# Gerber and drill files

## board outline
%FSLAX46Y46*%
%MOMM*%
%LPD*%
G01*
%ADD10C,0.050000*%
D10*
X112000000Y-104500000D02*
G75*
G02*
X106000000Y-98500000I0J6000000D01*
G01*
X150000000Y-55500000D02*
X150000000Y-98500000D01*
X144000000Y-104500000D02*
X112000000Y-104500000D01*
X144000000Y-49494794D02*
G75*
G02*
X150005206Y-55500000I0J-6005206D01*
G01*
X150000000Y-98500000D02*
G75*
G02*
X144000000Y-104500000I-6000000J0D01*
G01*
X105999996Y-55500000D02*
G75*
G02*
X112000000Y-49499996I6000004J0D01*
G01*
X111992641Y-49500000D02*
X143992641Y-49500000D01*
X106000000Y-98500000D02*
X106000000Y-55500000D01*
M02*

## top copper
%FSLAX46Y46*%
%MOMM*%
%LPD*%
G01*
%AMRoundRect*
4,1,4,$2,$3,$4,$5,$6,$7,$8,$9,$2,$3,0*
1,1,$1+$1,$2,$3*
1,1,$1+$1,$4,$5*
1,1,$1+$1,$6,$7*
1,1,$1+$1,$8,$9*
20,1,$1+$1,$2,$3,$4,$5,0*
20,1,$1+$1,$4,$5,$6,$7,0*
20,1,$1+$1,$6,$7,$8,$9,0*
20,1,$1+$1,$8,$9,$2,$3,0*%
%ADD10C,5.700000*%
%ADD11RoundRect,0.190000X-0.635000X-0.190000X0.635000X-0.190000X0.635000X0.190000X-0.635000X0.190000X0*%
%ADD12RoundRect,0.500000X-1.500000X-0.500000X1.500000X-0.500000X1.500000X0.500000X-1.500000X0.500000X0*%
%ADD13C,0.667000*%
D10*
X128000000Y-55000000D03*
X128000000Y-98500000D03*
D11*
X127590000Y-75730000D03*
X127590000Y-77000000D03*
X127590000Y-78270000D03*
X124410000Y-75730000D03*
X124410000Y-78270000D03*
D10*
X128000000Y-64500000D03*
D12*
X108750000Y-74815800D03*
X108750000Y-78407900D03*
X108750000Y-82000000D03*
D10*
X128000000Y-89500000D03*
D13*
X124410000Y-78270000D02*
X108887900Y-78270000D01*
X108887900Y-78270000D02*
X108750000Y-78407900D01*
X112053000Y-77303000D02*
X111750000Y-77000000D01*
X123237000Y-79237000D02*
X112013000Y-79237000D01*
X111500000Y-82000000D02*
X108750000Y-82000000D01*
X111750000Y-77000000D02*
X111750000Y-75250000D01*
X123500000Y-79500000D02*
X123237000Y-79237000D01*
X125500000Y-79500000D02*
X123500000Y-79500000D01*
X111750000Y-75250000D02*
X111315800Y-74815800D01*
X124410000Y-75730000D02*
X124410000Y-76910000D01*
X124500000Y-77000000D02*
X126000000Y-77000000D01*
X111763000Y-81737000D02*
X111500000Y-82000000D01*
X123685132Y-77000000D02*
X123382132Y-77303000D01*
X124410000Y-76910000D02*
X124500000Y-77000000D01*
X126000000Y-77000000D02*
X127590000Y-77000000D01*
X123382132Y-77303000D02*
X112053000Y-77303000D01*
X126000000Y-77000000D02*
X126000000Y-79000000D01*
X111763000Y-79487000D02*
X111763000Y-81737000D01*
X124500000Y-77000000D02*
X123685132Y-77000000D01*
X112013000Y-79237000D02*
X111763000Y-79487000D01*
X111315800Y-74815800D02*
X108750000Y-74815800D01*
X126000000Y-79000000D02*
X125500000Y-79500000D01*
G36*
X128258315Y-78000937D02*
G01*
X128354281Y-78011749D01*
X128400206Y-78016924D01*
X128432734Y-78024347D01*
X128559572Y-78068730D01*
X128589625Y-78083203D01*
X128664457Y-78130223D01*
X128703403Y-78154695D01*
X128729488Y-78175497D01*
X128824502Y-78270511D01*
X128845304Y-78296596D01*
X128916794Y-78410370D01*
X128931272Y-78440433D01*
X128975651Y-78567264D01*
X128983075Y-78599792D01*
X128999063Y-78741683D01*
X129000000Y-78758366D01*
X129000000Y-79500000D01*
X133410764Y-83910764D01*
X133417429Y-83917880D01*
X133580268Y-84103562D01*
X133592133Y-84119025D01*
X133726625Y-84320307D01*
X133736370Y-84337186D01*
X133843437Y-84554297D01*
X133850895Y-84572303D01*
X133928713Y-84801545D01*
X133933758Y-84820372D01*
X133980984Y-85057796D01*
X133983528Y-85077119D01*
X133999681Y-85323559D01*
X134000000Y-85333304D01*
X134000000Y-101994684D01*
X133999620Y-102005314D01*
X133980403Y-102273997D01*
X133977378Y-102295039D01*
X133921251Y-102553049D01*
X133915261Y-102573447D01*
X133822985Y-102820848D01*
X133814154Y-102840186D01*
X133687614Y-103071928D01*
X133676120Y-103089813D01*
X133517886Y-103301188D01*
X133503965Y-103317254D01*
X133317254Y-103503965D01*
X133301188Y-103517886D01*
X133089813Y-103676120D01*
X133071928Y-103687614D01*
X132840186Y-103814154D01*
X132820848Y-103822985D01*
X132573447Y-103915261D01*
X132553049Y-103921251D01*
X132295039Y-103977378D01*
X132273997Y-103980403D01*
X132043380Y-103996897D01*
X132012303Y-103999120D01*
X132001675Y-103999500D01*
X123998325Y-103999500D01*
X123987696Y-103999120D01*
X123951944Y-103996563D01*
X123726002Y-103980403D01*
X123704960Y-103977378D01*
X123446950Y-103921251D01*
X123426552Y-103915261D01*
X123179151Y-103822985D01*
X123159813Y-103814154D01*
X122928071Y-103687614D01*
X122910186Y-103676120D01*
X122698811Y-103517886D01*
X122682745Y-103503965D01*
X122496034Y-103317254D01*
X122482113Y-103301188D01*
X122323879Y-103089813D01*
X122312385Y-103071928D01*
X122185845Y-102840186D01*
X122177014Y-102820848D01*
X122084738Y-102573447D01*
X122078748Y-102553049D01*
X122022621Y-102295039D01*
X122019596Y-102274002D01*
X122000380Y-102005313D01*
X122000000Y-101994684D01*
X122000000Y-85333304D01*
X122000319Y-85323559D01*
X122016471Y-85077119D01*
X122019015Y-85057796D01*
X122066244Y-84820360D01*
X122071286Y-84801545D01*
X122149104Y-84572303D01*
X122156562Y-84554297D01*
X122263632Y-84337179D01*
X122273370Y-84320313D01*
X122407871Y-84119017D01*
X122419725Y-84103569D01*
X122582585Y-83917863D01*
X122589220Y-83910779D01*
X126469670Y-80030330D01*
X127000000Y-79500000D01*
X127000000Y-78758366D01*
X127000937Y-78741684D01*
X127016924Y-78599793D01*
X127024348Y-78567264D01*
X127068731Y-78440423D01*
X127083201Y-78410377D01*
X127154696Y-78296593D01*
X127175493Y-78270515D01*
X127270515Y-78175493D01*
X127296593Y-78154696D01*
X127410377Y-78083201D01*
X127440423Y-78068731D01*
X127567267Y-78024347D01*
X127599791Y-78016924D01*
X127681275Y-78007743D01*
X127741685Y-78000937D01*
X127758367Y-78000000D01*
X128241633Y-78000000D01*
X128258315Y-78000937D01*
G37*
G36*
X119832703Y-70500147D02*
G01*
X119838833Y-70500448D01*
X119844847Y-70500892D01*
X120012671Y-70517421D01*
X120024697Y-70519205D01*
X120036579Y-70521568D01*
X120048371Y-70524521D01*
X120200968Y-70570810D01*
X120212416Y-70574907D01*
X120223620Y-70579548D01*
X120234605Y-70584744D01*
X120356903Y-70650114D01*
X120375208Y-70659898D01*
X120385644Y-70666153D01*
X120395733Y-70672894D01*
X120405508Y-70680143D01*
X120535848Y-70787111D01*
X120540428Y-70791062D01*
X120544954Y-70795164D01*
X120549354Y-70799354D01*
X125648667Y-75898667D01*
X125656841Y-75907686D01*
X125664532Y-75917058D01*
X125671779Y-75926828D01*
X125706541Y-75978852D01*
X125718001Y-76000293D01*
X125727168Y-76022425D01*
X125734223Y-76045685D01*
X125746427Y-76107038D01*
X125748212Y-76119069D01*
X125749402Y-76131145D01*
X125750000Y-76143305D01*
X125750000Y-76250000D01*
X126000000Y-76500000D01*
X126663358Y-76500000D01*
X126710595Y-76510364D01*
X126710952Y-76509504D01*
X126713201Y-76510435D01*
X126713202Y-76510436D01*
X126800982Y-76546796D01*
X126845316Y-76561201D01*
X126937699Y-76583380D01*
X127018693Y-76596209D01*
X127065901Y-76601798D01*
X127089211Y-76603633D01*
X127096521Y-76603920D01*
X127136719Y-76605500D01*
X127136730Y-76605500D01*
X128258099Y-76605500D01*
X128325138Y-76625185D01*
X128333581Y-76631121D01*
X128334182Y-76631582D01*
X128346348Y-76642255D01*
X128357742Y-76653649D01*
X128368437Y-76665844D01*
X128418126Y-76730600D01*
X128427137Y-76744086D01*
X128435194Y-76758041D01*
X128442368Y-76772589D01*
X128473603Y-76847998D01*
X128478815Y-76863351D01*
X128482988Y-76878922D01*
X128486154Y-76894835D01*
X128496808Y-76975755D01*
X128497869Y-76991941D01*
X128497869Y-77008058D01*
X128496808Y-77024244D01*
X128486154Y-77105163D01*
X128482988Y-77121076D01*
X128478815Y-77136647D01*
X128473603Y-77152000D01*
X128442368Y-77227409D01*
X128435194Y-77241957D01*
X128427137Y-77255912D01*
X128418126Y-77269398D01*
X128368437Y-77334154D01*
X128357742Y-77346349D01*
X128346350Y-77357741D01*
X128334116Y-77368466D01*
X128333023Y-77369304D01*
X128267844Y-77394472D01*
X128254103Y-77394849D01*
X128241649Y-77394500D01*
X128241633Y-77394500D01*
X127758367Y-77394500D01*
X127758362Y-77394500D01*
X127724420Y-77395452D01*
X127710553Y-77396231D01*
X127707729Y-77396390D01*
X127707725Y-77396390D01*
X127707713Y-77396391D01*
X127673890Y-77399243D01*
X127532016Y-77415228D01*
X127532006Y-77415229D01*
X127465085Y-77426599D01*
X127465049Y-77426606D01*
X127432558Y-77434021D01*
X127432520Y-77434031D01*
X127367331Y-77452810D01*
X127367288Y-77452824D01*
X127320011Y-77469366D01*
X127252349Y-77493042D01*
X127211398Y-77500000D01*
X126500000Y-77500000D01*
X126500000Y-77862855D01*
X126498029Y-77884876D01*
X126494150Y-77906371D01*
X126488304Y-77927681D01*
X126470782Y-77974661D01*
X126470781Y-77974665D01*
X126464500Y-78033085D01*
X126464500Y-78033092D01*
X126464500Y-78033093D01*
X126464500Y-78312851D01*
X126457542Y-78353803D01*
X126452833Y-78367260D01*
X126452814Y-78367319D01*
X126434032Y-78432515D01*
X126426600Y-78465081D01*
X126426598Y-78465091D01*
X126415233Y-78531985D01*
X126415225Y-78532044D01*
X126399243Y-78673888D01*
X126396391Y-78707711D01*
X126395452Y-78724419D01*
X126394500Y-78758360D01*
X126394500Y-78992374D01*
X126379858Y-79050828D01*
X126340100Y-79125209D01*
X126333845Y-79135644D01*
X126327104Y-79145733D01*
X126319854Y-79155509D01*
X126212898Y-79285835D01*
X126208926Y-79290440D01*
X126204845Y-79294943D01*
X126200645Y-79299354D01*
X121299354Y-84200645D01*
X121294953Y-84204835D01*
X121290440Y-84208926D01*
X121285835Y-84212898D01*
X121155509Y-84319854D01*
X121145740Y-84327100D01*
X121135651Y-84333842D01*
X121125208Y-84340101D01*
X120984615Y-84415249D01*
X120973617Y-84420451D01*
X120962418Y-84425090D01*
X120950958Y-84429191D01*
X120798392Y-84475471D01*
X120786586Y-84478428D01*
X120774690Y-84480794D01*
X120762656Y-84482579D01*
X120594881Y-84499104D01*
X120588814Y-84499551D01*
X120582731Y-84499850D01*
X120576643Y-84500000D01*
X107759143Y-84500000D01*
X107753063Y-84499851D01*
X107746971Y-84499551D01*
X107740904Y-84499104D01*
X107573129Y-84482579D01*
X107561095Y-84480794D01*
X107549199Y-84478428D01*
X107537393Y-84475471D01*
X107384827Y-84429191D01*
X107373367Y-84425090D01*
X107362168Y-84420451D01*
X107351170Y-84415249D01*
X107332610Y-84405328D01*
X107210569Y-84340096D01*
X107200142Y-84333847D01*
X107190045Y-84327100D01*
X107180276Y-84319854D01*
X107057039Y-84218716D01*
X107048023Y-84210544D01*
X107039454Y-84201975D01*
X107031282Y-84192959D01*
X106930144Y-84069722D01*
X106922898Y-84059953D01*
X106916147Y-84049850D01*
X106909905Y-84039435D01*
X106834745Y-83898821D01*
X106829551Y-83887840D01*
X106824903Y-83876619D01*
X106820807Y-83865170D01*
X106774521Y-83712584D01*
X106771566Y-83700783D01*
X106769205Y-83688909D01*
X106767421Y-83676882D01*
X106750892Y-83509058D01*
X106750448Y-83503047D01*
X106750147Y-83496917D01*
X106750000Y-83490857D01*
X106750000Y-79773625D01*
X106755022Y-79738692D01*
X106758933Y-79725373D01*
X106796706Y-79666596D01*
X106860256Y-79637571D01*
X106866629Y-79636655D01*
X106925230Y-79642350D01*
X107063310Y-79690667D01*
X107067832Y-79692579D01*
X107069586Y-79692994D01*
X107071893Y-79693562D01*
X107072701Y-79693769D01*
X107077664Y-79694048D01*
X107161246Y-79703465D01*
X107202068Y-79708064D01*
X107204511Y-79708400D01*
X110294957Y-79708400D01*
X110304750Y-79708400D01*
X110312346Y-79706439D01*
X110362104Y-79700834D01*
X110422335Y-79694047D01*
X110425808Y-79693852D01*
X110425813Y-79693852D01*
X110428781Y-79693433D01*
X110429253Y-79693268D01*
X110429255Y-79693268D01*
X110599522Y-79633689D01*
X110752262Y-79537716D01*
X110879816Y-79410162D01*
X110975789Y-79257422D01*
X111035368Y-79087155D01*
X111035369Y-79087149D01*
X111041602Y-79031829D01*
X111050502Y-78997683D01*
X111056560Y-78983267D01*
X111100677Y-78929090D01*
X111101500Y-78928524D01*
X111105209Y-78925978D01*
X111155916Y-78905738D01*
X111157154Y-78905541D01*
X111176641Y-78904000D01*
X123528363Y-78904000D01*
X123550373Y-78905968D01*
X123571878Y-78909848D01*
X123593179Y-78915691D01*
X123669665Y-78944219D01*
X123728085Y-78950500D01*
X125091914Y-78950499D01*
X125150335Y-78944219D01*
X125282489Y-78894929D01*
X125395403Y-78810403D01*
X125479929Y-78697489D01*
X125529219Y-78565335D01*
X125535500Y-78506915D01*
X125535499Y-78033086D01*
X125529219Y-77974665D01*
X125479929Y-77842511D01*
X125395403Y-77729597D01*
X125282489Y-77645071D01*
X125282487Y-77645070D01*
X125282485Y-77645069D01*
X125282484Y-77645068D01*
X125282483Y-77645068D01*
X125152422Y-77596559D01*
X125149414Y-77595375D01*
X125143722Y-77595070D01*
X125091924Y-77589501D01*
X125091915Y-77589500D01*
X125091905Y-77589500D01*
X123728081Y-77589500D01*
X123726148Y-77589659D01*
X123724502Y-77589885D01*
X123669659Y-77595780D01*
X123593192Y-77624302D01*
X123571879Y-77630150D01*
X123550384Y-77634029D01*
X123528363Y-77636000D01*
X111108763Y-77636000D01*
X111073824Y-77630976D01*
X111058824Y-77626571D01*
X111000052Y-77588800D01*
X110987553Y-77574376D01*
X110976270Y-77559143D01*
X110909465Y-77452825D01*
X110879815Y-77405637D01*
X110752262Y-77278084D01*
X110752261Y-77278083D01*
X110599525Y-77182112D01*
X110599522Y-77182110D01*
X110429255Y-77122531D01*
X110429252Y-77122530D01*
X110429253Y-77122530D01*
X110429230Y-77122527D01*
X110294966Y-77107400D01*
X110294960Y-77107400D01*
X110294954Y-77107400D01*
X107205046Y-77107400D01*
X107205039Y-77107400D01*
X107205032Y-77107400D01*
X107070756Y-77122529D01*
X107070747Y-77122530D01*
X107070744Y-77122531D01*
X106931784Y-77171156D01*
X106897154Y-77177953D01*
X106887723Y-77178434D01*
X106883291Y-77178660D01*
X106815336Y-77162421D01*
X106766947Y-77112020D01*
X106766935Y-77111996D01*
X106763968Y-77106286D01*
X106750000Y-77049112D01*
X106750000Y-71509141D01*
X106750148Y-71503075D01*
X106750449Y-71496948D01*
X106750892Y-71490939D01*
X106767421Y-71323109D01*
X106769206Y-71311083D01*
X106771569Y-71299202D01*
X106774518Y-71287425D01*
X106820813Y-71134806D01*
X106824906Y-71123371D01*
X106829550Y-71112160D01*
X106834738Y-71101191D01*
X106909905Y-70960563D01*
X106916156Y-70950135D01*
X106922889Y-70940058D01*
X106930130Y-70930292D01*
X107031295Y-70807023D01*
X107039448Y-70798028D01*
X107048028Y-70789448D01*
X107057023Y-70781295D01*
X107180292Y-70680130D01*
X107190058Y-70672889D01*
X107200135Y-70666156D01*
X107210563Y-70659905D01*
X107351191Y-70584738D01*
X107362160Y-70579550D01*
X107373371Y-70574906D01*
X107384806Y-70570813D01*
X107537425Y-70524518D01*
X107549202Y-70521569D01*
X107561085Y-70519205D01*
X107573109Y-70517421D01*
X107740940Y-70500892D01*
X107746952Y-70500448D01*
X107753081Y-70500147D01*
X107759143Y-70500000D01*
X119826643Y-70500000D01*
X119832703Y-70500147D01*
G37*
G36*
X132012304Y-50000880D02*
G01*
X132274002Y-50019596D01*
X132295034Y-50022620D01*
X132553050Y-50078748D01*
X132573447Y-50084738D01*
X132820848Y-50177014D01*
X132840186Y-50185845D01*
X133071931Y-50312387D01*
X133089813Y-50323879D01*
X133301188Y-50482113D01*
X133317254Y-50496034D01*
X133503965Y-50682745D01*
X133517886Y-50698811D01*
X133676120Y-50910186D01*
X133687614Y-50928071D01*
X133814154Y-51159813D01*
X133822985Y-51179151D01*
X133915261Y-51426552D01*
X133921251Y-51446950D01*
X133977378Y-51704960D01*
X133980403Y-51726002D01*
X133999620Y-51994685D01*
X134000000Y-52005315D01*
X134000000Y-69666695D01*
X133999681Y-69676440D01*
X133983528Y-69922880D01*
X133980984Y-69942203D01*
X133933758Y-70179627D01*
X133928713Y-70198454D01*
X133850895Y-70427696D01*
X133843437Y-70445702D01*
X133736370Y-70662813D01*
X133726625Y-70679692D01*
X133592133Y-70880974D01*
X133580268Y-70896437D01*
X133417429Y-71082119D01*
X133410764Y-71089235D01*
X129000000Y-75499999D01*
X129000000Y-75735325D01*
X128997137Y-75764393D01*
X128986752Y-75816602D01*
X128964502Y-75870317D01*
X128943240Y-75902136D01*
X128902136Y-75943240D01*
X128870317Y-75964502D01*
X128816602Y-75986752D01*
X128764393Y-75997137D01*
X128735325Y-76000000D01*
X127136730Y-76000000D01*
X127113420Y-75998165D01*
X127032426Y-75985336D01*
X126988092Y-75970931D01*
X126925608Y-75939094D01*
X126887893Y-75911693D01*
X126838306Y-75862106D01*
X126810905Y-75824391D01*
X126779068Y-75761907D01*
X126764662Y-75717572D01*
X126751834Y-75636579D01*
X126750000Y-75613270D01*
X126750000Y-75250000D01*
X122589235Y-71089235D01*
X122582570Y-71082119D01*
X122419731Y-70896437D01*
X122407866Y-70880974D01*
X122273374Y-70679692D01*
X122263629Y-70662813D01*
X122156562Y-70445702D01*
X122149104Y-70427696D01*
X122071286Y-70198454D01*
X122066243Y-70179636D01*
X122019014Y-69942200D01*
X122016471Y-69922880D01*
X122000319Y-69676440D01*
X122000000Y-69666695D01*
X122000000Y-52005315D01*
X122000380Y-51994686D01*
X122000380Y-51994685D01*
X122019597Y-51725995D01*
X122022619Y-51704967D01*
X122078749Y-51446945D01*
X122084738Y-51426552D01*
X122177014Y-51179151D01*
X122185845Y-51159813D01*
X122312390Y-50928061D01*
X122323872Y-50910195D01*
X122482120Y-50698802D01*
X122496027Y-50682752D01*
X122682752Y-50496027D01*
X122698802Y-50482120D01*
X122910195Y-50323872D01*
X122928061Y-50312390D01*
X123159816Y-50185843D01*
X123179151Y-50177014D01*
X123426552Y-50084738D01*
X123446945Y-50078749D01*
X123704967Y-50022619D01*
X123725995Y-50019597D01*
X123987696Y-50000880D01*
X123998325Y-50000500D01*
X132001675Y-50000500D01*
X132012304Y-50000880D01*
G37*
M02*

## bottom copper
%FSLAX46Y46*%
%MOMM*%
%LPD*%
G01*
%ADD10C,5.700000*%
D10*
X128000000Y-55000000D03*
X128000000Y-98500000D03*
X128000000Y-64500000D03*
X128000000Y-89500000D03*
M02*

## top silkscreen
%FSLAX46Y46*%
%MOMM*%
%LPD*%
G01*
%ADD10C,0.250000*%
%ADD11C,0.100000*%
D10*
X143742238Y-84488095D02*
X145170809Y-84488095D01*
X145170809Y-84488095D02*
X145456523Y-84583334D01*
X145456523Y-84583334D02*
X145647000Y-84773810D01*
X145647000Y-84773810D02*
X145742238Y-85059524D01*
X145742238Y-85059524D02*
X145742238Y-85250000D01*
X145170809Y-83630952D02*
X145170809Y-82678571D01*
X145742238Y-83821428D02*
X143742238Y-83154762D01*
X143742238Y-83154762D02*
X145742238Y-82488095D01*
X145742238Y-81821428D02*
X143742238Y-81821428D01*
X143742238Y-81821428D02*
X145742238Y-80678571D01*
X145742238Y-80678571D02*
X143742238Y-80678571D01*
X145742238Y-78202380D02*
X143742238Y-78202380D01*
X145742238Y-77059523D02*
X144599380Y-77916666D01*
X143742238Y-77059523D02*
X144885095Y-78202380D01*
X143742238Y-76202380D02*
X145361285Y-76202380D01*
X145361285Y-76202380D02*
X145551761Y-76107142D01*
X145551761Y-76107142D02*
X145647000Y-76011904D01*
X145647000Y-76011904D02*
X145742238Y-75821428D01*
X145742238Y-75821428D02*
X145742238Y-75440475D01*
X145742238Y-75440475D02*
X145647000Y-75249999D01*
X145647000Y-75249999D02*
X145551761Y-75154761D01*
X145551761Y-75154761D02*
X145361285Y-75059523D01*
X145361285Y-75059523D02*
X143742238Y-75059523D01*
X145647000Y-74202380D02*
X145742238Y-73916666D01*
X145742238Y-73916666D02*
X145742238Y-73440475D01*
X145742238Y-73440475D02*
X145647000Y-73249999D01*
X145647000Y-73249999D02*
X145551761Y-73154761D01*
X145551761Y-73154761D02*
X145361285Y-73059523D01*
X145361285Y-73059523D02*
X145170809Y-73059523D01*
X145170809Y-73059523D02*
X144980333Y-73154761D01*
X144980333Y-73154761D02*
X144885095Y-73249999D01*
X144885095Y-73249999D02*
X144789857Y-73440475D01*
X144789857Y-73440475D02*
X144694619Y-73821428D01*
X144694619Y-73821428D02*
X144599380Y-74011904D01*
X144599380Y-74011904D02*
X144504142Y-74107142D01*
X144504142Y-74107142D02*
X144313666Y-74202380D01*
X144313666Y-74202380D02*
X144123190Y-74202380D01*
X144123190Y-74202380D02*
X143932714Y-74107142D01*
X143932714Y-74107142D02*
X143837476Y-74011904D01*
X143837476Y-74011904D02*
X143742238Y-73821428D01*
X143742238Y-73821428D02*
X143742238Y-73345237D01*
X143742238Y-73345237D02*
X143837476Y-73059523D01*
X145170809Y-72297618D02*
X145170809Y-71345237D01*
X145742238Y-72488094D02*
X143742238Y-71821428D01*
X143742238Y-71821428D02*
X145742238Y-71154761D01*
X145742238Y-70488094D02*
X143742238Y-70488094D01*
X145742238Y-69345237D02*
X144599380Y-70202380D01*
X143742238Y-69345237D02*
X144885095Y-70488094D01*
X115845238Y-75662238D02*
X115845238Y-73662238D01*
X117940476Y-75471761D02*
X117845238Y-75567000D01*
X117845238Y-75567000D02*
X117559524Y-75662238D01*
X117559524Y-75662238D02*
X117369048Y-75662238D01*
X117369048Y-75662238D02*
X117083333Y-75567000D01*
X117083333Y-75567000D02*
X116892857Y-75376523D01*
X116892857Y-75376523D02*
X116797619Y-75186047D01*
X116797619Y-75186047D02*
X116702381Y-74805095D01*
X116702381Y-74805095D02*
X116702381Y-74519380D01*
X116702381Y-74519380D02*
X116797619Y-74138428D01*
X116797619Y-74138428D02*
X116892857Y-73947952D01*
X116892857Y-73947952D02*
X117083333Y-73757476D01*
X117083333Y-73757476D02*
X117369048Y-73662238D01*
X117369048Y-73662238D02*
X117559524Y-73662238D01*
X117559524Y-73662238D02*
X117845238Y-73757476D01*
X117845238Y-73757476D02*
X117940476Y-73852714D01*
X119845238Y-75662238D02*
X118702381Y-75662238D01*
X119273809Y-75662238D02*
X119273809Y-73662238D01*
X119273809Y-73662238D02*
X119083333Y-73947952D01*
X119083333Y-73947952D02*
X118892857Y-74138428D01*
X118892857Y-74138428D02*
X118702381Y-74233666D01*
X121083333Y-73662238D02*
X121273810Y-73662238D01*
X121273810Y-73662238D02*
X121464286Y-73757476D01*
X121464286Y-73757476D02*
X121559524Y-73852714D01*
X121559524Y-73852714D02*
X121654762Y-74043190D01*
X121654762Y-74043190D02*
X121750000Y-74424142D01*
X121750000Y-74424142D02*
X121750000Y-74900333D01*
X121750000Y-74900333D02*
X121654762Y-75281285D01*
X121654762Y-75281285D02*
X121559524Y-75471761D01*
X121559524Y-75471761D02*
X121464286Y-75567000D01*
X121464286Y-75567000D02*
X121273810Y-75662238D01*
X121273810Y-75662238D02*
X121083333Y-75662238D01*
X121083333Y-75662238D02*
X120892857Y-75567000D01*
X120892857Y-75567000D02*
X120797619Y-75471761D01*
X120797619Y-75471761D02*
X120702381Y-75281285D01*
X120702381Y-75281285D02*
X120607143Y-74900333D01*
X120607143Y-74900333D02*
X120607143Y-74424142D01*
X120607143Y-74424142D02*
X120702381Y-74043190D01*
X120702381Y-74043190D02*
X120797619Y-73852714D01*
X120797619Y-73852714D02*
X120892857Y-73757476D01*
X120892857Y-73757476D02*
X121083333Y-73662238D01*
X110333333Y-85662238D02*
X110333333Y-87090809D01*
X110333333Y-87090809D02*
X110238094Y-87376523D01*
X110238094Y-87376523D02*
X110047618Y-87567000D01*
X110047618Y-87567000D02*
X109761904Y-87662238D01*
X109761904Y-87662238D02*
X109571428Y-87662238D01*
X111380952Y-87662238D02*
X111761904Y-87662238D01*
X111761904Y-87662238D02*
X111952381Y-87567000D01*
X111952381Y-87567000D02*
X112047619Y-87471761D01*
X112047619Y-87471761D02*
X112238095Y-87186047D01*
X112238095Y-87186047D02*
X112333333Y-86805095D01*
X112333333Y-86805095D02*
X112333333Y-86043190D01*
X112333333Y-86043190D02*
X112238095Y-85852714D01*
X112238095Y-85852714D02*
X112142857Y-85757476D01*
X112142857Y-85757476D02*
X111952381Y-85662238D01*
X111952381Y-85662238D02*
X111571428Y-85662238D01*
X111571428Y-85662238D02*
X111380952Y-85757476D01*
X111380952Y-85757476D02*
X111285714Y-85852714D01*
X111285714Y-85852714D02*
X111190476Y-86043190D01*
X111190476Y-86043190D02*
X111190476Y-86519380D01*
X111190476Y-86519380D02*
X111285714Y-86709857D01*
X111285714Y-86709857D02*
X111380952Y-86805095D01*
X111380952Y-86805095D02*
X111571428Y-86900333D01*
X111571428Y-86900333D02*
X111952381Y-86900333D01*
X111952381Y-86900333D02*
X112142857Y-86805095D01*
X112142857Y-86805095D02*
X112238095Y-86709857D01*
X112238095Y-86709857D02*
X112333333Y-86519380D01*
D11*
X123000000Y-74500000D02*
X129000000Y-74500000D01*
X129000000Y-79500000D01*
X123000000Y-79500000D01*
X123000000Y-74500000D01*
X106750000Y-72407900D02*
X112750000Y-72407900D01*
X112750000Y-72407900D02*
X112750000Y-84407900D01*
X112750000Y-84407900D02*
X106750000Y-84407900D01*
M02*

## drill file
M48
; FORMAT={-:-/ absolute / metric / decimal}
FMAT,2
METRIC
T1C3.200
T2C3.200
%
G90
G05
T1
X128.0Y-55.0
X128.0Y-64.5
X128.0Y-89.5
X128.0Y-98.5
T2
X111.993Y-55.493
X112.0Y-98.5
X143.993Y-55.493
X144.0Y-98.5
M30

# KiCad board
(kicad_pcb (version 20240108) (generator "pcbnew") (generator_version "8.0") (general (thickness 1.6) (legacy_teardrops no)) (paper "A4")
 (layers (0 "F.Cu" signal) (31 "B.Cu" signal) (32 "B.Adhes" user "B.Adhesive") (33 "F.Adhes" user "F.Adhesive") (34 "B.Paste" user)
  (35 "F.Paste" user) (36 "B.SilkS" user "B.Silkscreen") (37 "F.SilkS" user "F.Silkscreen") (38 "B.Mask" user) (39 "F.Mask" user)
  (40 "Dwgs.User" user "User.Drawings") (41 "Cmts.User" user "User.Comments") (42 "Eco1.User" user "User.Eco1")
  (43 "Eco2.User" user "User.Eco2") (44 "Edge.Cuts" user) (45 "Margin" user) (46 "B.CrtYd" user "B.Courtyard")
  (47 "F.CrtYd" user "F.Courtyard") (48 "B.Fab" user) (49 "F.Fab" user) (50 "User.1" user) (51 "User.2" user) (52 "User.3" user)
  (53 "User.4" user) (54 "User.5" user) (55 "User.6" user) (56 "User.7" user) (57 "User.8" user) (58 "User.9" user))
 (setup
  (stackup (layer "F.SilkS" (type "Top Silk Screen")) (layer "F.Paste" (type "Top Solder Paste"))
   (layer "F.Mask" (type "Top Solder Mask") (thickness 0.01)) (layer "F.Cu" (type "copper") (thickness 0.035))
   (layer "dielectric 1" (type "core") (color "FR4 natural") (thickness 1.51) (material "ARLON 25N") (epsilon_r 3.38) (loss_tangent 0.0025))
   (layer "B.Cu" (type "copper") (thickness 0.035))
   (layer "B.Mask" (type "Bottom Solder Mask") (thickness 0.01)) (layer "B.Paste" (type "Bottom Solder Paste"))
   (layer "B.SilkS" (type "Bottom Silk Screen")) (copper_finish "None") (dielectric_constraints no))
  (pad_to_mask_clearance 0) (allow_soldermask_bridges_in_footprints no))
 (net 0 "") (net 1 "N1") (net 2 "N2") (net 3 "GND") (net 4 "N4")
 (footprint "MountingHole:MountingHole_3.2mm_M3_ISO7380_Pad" (layer "F.Cu") (at 128 55)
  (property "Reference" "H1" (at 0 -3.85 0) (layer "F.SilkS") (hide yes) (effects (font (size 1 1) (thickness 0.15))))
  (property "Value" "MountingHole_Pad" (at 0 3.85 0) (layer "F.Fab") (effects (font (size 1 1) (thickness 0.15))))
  (pad "1" thru_hole circle (at 0 0) (size 5.7 5.7) (drill 3.2) (layers "*.Cu" "*.Mask") (remove_unused_layers no) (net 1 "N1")))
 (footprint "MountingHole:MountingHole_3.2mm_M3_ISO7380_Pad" (layer "F.Cu") (at 128 98.5)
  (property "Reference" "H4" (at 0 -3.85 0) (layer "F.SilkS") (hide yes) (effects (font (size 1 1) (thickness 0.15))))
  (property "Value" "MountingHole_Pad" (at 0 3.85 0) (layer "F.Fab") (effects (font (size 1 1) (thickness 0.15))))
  (pad "1" thru_hole circle (at 0 0) (size 5.7 5.7) (drill 3.2) (layers "*.Cu" "*.Mask") (remove_unused_layers no) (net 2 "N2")))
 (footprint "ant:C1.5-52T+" (layer "F.Cu") (at 126 77 -90)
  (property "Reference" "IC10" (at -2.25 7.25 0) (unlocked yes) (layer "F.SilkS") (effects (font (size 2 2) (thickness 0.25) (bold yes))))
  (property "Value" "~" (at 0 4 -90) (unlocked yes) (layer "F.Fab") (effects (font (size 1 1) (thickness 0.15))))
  (fp_rect (start -2.5 -3) (end 2.5 3) (stroke (width 0.1) (type default)) (fill none) (layer "F.SilkS"))
  (pad "1" smd roundrect (at -1.27 -1.59) (size 1.65 0.76) (layers "F.Cu" "F.Paste" "F.Mask") (roundrect_rratio 0.25) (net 1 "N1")
   (thermal_bridge_angle 45))
  (pad "2" smd roundrect (at 0 -1.59) (size 1.65 0.76) (layers "F.Cu" "F.Paste" "F.Mask") (roundrect_rratio 0.25) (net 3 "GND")
   (thermal_bridge_angle 45))
  (pad "3" smd roundrect (at 1.27 -1.59) (size 1.65 0.76) (layers "F.Cu" "F.Paste" "F.Mask") (roundrect_rratio 0.25) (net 2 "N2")
   (thermal_bridge_angle 45))
  (pad "4" smd roundrect (at -1.27 1.59) (size 1.65 0.76) (layers "F.Cu" "F.Paste" "F.Mask") (roundrect_rratio 0.25) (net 3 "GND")
   (thermal_bridge_angle 45))
  (pad "6" smd roundrect (at 1.27 1.59) (size 1.65 0.76) (layers "F.Cu" "F.Paste" "F.Mask") (roundrect_rratio 0.25) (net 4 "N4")
   (thermal_bridge_angle 45)))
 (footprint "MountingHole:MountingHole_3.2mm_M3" (layer "F.Cu") (at 112 98.5)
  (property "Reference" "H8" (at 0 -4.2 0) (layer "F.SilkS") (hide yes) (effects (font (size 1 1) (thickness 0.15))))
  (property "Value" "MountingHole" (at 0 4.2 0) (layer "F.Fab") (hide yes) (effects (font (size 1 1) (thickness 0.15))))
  (pad "" np_thru_hole circle (at 0 0) (size 3.2 3.2) (drill 3.2) (layers "*.Cu" "*.Mask")))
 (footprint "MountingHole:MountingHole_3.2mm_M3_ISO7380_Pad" (layer "F.Cu") (at 128 64.5)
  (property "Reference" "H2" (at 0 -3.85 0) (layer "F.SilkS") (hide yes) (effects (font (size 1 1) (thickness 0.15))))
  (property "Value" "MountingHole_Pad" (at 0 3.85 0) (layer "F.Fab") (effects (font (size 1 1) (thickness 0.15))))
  (pad "1" thru_hole circle (at 0 0) (size 5.7 5.7) (drill 3.2) (layers "*.Cu" "*.Mask") (remove_unused_layers no) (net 1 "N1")))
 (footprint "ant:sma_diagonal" (layer "F.Cu") (at 108.75 78.4079)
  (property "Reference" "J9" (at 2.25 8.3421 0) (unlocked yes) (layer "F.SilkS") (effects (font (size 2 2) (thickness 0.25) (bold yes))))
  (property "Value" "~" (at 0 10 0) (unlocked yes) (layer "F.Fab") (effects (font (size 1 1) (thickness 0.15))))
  (fp_line (start -2 -6) (end 4 -6) (stroke (width 0.1) (type default)) (layer "F.SilkS"))
  (fp_line (start 4 -6) (end 4 6) (stroke (width 0.1) (type default)) (layer "F.SilkS"))
  (fp_line (start 4 6) (end -2 6) (stroke (width 0.1) (type default)) (layer "F.SilkS"))
  (pad "1" smd roundrect (at 0 -3.5921) (size 4 2) (layers "F.Cu" "F.Paste" "F.Mask") (roundrect_rratio 0.25) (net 3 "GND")
   (thermal_bridge_angle 45))
  (pad "2" smd roundrect (at 0 0) (size 4 2) (layers "F.Cu" "F.Paste" "F.Mask") (roundrect_rratio 0.25) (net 4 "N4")
   (thermal_bridge_angle 45))
  (pad "3" smd roundrect (at 0 3.5921) (size 4 2) (layers "F.Cu" "F.Paste" "F.Mask") (roundrect_rratio 0.25) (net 3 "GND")
   (thermal_bridge_angle 45)))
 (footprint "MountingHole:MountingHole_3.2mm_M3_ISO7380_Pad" (layer "F.Cu") (at 128 89.5)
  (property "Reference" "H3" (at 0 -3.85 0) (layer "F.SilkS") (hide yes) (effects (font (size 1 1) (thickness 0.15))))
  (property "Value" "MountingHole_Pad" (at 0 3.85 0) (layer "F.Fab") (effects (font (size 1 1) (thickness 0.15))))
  (pad "1" thru_hole circle (at 0 0) (size 5.7 5.7) (drill 3.2) (layers "*.Cu" "*.Mask") (remove_unused_layers no) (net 2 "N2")))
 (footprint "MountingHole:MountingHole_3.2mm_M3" (layer "F.Cu") (at 144 98.5)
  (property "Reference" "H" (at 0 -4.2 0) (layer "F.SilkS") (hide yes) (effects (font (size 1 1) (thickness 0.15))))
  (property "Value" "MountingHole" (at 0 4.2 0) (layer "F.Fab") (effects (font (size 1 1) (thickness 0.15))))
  (pad "" np_thru_hole circle (at 0 0) (size 3.2 3.2) (drill 3.2) (layers "*.Cu" "*.Mask")))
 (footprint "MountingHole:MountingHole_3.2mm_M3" (layer "F.Cu") (at 111.992641 55.492641)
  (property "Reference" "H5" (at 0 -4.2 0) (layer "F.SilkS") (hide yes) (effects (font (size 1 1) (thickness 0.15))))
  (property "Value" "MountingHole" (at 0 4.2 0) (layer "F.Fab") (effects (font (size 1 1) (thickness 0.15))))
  (pad "" np_thru_hole circle (at 0 0) (size 3.2 3.2) (drill 3.2) (layers "*.Cu" "*.Mask")))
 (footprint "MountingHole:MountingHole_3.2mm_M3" (layer "F.Cu") (at 143.992641 55.492641)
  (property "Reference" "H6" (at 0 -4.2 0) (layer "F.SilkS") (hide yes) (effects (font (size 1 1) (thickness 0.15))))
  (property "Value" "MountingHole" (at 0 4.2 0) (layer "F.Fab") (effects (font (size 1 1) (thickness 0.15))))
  (pad "" np_thru_hole circle (at 0 0) (size 3.2 3.2) (drill 3.2) (layers "*.Cu" "*.Mask")))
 (gr_arc (start 112 104.5) (mid 107.757359 102.742641) (end 106 98.5) (stroke (width 0.05) (type default)) (layer "Edge.Cuts"))
 (gr_line (start 150 55.5) (end 150 98.5) (stroke (width 0.05) (type default)) (layer "Edge.Cuts"))
 (gr_line (start 144 104.5) (end 112 104.5) (stroke (width 0.05) (type default)) (layer "Edge.Cuts"))
 (gr_arc (start 144 49.494794) (mid 148.246322 51.253678) (end 150.005206 55.5) (stroke (width 0.05) (type default)) (layer "Edge.Cuts"))
 (gr_arc (start 150 98.5) (mid 148.242641 102.742641) (end 144 104.5) (stroke (width 0.05) (type default)) (layer "Edge.Cuts"))
 (gr_arc (start 105.999996 55.5) (mid 107.757356 51.257356) (end 112 49.499996) (stroke (width 0.05) (type default)) (layer "Edge.Cuts"))
 (gr_line (start 111.992641 49.5) (end 143.992641 49.5) (stroke (width 0.05) (type default)) (layer "Edge.Cuts"))
 (gr_line (start 106 98.5) (end 106 55.5) (stroke (width 0.05) (type default)) (layer "Edge.Cuts"))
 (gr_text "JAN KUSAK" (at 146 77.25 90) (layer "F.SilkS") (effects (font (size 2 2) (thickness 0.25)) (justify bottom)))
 (segment (start 124.41 78.27) (end 108.8879 78.27) (width 0.667) (layer "F.Cu") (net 4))
 (segment (start 108.8879 78.27) (end 108.75 78.4079) (width 0.667) (layer "F.Cu") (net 4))
 (segment (start 112.053 77.303) (end 111.75 77) (width 0.667) (layer "F.Cu") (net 3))
 (segment (start 123.237 79.237) (end 112.013 79.237) (width 0.667) (layer "F.Cu") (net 3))
 (segment (start 111.5 82) (end 108.75 82) (width 0.667) (layer "F.Cu") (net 3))
 (segment (start 111.75 77) (end 111.75 75.25) (width 0.667) (layer "F.Cu") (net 3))
 (segment (start 123.5 79.5) (end 123.237 79.237) (width 0.667) (layer "F.Cu") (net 3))
 (segment (start 125.5 79.5) (end 123.5 79.5) (width 0.667) (layer "F.Cu") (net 3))
 (segment (start 111.75 75.25) (end 111.3158 74.8158) (width 0.667) (layer "F.Cu") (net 3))
 (segment (start 124.41 75.73) (end 124.41 76.91) (width 0.667) (layer "F.Cu") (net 3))
 (segment (start 124.5 77) (end 126 77) (width 0.667) (layer "F.Cu") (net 3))
 (segment (start 111.763 81.737) (end 111.5 82) (width 0.667) (layer "F.Cu") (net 3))
 (segment (start 123.685132 77) (end 123.382132 77.303) (width 0.667) (layer "F.Cu") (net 3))
 (segment (start 124.41 76.91) (end 124.5 77) (width 0.667) (layer "F.Cu") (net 3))
 (segment (start 126 77) (end 127.59 77) (width 0.667) (layer "F.Cu") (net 3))
 (segment (start 123.382132 77.303) (end 112.053 77.303) (width 0.667) (layer "F.Cu") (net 3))
 (segment (start 126 77) (end 126 79) (width 0.667) (layer "F.Cu") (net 3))
 (segment (start 111.763 79.487) (end 111.763 81.737) (width 0.667) (layer "F.Cu") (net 3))
 (segment (start 124.5 77) (end 123.685132 77) (width 0.667) (layer "F.Cu") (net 3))
 (segment (start 112.013 79.237) (end 111.763 79.487) (width 0.667) (layer "F.Cu") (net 3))
 (segment (start 111.3158 74.8158) (end 108.75 74.8158) (width 0.667) (layer "F.Cu") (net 3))
 (segment (start 126 79) (end 125.5 79.5) (width 0.667) (layer "F.Cu") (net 3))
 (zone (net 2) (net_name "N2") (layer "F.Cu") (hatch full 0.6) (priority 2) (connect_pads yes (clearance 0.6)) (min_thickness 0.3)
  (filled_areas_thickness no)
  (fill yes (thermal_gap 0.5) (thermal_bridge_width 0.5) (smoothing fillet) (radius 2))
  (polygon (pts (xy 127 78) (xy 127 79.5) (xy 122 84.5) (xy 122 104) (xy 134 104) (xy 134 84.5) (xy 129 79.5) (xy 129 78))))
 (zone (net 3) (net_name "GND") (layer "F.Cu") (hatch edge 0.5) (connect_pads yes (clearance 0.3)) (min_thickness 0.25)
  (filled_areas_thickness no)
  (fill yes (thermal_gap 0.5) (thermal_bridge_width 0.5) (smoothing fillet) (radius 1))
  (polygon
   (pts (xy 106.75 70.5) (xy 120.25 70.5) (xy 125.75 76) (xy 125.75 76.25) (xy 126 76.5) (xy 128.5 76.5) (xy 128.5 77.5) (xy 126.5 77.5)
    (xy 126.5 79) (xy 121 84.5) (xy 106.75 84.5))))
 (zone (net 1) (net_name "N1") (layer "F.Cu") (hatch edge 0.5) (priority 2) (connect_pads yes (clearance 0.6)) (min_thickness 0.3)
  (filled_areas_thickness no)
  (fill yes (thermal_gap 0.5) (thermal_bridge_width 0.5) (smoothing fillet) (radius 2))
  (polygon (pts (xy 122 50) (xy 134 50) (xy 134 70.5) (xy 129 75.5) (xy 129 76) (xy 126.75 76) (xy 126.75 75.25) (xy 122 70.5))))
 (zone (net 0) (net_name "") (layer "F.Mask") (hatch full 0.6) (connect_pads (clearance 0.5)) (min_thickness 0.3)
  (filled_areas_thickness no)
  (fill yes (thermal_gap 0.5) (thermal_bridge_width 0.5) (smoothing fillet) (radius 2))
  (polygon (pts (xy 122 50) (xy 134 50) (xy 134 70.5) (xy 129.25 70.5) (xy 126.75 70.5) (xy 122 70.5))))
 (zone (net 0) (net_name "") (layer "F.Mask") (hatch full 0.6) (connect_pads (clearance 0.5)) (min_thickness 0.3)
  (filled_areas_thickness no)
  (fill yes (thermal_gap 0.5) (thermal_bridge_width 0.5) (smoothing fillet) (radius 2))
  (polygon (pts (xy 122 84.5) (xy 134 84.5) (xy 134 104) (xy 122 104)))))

